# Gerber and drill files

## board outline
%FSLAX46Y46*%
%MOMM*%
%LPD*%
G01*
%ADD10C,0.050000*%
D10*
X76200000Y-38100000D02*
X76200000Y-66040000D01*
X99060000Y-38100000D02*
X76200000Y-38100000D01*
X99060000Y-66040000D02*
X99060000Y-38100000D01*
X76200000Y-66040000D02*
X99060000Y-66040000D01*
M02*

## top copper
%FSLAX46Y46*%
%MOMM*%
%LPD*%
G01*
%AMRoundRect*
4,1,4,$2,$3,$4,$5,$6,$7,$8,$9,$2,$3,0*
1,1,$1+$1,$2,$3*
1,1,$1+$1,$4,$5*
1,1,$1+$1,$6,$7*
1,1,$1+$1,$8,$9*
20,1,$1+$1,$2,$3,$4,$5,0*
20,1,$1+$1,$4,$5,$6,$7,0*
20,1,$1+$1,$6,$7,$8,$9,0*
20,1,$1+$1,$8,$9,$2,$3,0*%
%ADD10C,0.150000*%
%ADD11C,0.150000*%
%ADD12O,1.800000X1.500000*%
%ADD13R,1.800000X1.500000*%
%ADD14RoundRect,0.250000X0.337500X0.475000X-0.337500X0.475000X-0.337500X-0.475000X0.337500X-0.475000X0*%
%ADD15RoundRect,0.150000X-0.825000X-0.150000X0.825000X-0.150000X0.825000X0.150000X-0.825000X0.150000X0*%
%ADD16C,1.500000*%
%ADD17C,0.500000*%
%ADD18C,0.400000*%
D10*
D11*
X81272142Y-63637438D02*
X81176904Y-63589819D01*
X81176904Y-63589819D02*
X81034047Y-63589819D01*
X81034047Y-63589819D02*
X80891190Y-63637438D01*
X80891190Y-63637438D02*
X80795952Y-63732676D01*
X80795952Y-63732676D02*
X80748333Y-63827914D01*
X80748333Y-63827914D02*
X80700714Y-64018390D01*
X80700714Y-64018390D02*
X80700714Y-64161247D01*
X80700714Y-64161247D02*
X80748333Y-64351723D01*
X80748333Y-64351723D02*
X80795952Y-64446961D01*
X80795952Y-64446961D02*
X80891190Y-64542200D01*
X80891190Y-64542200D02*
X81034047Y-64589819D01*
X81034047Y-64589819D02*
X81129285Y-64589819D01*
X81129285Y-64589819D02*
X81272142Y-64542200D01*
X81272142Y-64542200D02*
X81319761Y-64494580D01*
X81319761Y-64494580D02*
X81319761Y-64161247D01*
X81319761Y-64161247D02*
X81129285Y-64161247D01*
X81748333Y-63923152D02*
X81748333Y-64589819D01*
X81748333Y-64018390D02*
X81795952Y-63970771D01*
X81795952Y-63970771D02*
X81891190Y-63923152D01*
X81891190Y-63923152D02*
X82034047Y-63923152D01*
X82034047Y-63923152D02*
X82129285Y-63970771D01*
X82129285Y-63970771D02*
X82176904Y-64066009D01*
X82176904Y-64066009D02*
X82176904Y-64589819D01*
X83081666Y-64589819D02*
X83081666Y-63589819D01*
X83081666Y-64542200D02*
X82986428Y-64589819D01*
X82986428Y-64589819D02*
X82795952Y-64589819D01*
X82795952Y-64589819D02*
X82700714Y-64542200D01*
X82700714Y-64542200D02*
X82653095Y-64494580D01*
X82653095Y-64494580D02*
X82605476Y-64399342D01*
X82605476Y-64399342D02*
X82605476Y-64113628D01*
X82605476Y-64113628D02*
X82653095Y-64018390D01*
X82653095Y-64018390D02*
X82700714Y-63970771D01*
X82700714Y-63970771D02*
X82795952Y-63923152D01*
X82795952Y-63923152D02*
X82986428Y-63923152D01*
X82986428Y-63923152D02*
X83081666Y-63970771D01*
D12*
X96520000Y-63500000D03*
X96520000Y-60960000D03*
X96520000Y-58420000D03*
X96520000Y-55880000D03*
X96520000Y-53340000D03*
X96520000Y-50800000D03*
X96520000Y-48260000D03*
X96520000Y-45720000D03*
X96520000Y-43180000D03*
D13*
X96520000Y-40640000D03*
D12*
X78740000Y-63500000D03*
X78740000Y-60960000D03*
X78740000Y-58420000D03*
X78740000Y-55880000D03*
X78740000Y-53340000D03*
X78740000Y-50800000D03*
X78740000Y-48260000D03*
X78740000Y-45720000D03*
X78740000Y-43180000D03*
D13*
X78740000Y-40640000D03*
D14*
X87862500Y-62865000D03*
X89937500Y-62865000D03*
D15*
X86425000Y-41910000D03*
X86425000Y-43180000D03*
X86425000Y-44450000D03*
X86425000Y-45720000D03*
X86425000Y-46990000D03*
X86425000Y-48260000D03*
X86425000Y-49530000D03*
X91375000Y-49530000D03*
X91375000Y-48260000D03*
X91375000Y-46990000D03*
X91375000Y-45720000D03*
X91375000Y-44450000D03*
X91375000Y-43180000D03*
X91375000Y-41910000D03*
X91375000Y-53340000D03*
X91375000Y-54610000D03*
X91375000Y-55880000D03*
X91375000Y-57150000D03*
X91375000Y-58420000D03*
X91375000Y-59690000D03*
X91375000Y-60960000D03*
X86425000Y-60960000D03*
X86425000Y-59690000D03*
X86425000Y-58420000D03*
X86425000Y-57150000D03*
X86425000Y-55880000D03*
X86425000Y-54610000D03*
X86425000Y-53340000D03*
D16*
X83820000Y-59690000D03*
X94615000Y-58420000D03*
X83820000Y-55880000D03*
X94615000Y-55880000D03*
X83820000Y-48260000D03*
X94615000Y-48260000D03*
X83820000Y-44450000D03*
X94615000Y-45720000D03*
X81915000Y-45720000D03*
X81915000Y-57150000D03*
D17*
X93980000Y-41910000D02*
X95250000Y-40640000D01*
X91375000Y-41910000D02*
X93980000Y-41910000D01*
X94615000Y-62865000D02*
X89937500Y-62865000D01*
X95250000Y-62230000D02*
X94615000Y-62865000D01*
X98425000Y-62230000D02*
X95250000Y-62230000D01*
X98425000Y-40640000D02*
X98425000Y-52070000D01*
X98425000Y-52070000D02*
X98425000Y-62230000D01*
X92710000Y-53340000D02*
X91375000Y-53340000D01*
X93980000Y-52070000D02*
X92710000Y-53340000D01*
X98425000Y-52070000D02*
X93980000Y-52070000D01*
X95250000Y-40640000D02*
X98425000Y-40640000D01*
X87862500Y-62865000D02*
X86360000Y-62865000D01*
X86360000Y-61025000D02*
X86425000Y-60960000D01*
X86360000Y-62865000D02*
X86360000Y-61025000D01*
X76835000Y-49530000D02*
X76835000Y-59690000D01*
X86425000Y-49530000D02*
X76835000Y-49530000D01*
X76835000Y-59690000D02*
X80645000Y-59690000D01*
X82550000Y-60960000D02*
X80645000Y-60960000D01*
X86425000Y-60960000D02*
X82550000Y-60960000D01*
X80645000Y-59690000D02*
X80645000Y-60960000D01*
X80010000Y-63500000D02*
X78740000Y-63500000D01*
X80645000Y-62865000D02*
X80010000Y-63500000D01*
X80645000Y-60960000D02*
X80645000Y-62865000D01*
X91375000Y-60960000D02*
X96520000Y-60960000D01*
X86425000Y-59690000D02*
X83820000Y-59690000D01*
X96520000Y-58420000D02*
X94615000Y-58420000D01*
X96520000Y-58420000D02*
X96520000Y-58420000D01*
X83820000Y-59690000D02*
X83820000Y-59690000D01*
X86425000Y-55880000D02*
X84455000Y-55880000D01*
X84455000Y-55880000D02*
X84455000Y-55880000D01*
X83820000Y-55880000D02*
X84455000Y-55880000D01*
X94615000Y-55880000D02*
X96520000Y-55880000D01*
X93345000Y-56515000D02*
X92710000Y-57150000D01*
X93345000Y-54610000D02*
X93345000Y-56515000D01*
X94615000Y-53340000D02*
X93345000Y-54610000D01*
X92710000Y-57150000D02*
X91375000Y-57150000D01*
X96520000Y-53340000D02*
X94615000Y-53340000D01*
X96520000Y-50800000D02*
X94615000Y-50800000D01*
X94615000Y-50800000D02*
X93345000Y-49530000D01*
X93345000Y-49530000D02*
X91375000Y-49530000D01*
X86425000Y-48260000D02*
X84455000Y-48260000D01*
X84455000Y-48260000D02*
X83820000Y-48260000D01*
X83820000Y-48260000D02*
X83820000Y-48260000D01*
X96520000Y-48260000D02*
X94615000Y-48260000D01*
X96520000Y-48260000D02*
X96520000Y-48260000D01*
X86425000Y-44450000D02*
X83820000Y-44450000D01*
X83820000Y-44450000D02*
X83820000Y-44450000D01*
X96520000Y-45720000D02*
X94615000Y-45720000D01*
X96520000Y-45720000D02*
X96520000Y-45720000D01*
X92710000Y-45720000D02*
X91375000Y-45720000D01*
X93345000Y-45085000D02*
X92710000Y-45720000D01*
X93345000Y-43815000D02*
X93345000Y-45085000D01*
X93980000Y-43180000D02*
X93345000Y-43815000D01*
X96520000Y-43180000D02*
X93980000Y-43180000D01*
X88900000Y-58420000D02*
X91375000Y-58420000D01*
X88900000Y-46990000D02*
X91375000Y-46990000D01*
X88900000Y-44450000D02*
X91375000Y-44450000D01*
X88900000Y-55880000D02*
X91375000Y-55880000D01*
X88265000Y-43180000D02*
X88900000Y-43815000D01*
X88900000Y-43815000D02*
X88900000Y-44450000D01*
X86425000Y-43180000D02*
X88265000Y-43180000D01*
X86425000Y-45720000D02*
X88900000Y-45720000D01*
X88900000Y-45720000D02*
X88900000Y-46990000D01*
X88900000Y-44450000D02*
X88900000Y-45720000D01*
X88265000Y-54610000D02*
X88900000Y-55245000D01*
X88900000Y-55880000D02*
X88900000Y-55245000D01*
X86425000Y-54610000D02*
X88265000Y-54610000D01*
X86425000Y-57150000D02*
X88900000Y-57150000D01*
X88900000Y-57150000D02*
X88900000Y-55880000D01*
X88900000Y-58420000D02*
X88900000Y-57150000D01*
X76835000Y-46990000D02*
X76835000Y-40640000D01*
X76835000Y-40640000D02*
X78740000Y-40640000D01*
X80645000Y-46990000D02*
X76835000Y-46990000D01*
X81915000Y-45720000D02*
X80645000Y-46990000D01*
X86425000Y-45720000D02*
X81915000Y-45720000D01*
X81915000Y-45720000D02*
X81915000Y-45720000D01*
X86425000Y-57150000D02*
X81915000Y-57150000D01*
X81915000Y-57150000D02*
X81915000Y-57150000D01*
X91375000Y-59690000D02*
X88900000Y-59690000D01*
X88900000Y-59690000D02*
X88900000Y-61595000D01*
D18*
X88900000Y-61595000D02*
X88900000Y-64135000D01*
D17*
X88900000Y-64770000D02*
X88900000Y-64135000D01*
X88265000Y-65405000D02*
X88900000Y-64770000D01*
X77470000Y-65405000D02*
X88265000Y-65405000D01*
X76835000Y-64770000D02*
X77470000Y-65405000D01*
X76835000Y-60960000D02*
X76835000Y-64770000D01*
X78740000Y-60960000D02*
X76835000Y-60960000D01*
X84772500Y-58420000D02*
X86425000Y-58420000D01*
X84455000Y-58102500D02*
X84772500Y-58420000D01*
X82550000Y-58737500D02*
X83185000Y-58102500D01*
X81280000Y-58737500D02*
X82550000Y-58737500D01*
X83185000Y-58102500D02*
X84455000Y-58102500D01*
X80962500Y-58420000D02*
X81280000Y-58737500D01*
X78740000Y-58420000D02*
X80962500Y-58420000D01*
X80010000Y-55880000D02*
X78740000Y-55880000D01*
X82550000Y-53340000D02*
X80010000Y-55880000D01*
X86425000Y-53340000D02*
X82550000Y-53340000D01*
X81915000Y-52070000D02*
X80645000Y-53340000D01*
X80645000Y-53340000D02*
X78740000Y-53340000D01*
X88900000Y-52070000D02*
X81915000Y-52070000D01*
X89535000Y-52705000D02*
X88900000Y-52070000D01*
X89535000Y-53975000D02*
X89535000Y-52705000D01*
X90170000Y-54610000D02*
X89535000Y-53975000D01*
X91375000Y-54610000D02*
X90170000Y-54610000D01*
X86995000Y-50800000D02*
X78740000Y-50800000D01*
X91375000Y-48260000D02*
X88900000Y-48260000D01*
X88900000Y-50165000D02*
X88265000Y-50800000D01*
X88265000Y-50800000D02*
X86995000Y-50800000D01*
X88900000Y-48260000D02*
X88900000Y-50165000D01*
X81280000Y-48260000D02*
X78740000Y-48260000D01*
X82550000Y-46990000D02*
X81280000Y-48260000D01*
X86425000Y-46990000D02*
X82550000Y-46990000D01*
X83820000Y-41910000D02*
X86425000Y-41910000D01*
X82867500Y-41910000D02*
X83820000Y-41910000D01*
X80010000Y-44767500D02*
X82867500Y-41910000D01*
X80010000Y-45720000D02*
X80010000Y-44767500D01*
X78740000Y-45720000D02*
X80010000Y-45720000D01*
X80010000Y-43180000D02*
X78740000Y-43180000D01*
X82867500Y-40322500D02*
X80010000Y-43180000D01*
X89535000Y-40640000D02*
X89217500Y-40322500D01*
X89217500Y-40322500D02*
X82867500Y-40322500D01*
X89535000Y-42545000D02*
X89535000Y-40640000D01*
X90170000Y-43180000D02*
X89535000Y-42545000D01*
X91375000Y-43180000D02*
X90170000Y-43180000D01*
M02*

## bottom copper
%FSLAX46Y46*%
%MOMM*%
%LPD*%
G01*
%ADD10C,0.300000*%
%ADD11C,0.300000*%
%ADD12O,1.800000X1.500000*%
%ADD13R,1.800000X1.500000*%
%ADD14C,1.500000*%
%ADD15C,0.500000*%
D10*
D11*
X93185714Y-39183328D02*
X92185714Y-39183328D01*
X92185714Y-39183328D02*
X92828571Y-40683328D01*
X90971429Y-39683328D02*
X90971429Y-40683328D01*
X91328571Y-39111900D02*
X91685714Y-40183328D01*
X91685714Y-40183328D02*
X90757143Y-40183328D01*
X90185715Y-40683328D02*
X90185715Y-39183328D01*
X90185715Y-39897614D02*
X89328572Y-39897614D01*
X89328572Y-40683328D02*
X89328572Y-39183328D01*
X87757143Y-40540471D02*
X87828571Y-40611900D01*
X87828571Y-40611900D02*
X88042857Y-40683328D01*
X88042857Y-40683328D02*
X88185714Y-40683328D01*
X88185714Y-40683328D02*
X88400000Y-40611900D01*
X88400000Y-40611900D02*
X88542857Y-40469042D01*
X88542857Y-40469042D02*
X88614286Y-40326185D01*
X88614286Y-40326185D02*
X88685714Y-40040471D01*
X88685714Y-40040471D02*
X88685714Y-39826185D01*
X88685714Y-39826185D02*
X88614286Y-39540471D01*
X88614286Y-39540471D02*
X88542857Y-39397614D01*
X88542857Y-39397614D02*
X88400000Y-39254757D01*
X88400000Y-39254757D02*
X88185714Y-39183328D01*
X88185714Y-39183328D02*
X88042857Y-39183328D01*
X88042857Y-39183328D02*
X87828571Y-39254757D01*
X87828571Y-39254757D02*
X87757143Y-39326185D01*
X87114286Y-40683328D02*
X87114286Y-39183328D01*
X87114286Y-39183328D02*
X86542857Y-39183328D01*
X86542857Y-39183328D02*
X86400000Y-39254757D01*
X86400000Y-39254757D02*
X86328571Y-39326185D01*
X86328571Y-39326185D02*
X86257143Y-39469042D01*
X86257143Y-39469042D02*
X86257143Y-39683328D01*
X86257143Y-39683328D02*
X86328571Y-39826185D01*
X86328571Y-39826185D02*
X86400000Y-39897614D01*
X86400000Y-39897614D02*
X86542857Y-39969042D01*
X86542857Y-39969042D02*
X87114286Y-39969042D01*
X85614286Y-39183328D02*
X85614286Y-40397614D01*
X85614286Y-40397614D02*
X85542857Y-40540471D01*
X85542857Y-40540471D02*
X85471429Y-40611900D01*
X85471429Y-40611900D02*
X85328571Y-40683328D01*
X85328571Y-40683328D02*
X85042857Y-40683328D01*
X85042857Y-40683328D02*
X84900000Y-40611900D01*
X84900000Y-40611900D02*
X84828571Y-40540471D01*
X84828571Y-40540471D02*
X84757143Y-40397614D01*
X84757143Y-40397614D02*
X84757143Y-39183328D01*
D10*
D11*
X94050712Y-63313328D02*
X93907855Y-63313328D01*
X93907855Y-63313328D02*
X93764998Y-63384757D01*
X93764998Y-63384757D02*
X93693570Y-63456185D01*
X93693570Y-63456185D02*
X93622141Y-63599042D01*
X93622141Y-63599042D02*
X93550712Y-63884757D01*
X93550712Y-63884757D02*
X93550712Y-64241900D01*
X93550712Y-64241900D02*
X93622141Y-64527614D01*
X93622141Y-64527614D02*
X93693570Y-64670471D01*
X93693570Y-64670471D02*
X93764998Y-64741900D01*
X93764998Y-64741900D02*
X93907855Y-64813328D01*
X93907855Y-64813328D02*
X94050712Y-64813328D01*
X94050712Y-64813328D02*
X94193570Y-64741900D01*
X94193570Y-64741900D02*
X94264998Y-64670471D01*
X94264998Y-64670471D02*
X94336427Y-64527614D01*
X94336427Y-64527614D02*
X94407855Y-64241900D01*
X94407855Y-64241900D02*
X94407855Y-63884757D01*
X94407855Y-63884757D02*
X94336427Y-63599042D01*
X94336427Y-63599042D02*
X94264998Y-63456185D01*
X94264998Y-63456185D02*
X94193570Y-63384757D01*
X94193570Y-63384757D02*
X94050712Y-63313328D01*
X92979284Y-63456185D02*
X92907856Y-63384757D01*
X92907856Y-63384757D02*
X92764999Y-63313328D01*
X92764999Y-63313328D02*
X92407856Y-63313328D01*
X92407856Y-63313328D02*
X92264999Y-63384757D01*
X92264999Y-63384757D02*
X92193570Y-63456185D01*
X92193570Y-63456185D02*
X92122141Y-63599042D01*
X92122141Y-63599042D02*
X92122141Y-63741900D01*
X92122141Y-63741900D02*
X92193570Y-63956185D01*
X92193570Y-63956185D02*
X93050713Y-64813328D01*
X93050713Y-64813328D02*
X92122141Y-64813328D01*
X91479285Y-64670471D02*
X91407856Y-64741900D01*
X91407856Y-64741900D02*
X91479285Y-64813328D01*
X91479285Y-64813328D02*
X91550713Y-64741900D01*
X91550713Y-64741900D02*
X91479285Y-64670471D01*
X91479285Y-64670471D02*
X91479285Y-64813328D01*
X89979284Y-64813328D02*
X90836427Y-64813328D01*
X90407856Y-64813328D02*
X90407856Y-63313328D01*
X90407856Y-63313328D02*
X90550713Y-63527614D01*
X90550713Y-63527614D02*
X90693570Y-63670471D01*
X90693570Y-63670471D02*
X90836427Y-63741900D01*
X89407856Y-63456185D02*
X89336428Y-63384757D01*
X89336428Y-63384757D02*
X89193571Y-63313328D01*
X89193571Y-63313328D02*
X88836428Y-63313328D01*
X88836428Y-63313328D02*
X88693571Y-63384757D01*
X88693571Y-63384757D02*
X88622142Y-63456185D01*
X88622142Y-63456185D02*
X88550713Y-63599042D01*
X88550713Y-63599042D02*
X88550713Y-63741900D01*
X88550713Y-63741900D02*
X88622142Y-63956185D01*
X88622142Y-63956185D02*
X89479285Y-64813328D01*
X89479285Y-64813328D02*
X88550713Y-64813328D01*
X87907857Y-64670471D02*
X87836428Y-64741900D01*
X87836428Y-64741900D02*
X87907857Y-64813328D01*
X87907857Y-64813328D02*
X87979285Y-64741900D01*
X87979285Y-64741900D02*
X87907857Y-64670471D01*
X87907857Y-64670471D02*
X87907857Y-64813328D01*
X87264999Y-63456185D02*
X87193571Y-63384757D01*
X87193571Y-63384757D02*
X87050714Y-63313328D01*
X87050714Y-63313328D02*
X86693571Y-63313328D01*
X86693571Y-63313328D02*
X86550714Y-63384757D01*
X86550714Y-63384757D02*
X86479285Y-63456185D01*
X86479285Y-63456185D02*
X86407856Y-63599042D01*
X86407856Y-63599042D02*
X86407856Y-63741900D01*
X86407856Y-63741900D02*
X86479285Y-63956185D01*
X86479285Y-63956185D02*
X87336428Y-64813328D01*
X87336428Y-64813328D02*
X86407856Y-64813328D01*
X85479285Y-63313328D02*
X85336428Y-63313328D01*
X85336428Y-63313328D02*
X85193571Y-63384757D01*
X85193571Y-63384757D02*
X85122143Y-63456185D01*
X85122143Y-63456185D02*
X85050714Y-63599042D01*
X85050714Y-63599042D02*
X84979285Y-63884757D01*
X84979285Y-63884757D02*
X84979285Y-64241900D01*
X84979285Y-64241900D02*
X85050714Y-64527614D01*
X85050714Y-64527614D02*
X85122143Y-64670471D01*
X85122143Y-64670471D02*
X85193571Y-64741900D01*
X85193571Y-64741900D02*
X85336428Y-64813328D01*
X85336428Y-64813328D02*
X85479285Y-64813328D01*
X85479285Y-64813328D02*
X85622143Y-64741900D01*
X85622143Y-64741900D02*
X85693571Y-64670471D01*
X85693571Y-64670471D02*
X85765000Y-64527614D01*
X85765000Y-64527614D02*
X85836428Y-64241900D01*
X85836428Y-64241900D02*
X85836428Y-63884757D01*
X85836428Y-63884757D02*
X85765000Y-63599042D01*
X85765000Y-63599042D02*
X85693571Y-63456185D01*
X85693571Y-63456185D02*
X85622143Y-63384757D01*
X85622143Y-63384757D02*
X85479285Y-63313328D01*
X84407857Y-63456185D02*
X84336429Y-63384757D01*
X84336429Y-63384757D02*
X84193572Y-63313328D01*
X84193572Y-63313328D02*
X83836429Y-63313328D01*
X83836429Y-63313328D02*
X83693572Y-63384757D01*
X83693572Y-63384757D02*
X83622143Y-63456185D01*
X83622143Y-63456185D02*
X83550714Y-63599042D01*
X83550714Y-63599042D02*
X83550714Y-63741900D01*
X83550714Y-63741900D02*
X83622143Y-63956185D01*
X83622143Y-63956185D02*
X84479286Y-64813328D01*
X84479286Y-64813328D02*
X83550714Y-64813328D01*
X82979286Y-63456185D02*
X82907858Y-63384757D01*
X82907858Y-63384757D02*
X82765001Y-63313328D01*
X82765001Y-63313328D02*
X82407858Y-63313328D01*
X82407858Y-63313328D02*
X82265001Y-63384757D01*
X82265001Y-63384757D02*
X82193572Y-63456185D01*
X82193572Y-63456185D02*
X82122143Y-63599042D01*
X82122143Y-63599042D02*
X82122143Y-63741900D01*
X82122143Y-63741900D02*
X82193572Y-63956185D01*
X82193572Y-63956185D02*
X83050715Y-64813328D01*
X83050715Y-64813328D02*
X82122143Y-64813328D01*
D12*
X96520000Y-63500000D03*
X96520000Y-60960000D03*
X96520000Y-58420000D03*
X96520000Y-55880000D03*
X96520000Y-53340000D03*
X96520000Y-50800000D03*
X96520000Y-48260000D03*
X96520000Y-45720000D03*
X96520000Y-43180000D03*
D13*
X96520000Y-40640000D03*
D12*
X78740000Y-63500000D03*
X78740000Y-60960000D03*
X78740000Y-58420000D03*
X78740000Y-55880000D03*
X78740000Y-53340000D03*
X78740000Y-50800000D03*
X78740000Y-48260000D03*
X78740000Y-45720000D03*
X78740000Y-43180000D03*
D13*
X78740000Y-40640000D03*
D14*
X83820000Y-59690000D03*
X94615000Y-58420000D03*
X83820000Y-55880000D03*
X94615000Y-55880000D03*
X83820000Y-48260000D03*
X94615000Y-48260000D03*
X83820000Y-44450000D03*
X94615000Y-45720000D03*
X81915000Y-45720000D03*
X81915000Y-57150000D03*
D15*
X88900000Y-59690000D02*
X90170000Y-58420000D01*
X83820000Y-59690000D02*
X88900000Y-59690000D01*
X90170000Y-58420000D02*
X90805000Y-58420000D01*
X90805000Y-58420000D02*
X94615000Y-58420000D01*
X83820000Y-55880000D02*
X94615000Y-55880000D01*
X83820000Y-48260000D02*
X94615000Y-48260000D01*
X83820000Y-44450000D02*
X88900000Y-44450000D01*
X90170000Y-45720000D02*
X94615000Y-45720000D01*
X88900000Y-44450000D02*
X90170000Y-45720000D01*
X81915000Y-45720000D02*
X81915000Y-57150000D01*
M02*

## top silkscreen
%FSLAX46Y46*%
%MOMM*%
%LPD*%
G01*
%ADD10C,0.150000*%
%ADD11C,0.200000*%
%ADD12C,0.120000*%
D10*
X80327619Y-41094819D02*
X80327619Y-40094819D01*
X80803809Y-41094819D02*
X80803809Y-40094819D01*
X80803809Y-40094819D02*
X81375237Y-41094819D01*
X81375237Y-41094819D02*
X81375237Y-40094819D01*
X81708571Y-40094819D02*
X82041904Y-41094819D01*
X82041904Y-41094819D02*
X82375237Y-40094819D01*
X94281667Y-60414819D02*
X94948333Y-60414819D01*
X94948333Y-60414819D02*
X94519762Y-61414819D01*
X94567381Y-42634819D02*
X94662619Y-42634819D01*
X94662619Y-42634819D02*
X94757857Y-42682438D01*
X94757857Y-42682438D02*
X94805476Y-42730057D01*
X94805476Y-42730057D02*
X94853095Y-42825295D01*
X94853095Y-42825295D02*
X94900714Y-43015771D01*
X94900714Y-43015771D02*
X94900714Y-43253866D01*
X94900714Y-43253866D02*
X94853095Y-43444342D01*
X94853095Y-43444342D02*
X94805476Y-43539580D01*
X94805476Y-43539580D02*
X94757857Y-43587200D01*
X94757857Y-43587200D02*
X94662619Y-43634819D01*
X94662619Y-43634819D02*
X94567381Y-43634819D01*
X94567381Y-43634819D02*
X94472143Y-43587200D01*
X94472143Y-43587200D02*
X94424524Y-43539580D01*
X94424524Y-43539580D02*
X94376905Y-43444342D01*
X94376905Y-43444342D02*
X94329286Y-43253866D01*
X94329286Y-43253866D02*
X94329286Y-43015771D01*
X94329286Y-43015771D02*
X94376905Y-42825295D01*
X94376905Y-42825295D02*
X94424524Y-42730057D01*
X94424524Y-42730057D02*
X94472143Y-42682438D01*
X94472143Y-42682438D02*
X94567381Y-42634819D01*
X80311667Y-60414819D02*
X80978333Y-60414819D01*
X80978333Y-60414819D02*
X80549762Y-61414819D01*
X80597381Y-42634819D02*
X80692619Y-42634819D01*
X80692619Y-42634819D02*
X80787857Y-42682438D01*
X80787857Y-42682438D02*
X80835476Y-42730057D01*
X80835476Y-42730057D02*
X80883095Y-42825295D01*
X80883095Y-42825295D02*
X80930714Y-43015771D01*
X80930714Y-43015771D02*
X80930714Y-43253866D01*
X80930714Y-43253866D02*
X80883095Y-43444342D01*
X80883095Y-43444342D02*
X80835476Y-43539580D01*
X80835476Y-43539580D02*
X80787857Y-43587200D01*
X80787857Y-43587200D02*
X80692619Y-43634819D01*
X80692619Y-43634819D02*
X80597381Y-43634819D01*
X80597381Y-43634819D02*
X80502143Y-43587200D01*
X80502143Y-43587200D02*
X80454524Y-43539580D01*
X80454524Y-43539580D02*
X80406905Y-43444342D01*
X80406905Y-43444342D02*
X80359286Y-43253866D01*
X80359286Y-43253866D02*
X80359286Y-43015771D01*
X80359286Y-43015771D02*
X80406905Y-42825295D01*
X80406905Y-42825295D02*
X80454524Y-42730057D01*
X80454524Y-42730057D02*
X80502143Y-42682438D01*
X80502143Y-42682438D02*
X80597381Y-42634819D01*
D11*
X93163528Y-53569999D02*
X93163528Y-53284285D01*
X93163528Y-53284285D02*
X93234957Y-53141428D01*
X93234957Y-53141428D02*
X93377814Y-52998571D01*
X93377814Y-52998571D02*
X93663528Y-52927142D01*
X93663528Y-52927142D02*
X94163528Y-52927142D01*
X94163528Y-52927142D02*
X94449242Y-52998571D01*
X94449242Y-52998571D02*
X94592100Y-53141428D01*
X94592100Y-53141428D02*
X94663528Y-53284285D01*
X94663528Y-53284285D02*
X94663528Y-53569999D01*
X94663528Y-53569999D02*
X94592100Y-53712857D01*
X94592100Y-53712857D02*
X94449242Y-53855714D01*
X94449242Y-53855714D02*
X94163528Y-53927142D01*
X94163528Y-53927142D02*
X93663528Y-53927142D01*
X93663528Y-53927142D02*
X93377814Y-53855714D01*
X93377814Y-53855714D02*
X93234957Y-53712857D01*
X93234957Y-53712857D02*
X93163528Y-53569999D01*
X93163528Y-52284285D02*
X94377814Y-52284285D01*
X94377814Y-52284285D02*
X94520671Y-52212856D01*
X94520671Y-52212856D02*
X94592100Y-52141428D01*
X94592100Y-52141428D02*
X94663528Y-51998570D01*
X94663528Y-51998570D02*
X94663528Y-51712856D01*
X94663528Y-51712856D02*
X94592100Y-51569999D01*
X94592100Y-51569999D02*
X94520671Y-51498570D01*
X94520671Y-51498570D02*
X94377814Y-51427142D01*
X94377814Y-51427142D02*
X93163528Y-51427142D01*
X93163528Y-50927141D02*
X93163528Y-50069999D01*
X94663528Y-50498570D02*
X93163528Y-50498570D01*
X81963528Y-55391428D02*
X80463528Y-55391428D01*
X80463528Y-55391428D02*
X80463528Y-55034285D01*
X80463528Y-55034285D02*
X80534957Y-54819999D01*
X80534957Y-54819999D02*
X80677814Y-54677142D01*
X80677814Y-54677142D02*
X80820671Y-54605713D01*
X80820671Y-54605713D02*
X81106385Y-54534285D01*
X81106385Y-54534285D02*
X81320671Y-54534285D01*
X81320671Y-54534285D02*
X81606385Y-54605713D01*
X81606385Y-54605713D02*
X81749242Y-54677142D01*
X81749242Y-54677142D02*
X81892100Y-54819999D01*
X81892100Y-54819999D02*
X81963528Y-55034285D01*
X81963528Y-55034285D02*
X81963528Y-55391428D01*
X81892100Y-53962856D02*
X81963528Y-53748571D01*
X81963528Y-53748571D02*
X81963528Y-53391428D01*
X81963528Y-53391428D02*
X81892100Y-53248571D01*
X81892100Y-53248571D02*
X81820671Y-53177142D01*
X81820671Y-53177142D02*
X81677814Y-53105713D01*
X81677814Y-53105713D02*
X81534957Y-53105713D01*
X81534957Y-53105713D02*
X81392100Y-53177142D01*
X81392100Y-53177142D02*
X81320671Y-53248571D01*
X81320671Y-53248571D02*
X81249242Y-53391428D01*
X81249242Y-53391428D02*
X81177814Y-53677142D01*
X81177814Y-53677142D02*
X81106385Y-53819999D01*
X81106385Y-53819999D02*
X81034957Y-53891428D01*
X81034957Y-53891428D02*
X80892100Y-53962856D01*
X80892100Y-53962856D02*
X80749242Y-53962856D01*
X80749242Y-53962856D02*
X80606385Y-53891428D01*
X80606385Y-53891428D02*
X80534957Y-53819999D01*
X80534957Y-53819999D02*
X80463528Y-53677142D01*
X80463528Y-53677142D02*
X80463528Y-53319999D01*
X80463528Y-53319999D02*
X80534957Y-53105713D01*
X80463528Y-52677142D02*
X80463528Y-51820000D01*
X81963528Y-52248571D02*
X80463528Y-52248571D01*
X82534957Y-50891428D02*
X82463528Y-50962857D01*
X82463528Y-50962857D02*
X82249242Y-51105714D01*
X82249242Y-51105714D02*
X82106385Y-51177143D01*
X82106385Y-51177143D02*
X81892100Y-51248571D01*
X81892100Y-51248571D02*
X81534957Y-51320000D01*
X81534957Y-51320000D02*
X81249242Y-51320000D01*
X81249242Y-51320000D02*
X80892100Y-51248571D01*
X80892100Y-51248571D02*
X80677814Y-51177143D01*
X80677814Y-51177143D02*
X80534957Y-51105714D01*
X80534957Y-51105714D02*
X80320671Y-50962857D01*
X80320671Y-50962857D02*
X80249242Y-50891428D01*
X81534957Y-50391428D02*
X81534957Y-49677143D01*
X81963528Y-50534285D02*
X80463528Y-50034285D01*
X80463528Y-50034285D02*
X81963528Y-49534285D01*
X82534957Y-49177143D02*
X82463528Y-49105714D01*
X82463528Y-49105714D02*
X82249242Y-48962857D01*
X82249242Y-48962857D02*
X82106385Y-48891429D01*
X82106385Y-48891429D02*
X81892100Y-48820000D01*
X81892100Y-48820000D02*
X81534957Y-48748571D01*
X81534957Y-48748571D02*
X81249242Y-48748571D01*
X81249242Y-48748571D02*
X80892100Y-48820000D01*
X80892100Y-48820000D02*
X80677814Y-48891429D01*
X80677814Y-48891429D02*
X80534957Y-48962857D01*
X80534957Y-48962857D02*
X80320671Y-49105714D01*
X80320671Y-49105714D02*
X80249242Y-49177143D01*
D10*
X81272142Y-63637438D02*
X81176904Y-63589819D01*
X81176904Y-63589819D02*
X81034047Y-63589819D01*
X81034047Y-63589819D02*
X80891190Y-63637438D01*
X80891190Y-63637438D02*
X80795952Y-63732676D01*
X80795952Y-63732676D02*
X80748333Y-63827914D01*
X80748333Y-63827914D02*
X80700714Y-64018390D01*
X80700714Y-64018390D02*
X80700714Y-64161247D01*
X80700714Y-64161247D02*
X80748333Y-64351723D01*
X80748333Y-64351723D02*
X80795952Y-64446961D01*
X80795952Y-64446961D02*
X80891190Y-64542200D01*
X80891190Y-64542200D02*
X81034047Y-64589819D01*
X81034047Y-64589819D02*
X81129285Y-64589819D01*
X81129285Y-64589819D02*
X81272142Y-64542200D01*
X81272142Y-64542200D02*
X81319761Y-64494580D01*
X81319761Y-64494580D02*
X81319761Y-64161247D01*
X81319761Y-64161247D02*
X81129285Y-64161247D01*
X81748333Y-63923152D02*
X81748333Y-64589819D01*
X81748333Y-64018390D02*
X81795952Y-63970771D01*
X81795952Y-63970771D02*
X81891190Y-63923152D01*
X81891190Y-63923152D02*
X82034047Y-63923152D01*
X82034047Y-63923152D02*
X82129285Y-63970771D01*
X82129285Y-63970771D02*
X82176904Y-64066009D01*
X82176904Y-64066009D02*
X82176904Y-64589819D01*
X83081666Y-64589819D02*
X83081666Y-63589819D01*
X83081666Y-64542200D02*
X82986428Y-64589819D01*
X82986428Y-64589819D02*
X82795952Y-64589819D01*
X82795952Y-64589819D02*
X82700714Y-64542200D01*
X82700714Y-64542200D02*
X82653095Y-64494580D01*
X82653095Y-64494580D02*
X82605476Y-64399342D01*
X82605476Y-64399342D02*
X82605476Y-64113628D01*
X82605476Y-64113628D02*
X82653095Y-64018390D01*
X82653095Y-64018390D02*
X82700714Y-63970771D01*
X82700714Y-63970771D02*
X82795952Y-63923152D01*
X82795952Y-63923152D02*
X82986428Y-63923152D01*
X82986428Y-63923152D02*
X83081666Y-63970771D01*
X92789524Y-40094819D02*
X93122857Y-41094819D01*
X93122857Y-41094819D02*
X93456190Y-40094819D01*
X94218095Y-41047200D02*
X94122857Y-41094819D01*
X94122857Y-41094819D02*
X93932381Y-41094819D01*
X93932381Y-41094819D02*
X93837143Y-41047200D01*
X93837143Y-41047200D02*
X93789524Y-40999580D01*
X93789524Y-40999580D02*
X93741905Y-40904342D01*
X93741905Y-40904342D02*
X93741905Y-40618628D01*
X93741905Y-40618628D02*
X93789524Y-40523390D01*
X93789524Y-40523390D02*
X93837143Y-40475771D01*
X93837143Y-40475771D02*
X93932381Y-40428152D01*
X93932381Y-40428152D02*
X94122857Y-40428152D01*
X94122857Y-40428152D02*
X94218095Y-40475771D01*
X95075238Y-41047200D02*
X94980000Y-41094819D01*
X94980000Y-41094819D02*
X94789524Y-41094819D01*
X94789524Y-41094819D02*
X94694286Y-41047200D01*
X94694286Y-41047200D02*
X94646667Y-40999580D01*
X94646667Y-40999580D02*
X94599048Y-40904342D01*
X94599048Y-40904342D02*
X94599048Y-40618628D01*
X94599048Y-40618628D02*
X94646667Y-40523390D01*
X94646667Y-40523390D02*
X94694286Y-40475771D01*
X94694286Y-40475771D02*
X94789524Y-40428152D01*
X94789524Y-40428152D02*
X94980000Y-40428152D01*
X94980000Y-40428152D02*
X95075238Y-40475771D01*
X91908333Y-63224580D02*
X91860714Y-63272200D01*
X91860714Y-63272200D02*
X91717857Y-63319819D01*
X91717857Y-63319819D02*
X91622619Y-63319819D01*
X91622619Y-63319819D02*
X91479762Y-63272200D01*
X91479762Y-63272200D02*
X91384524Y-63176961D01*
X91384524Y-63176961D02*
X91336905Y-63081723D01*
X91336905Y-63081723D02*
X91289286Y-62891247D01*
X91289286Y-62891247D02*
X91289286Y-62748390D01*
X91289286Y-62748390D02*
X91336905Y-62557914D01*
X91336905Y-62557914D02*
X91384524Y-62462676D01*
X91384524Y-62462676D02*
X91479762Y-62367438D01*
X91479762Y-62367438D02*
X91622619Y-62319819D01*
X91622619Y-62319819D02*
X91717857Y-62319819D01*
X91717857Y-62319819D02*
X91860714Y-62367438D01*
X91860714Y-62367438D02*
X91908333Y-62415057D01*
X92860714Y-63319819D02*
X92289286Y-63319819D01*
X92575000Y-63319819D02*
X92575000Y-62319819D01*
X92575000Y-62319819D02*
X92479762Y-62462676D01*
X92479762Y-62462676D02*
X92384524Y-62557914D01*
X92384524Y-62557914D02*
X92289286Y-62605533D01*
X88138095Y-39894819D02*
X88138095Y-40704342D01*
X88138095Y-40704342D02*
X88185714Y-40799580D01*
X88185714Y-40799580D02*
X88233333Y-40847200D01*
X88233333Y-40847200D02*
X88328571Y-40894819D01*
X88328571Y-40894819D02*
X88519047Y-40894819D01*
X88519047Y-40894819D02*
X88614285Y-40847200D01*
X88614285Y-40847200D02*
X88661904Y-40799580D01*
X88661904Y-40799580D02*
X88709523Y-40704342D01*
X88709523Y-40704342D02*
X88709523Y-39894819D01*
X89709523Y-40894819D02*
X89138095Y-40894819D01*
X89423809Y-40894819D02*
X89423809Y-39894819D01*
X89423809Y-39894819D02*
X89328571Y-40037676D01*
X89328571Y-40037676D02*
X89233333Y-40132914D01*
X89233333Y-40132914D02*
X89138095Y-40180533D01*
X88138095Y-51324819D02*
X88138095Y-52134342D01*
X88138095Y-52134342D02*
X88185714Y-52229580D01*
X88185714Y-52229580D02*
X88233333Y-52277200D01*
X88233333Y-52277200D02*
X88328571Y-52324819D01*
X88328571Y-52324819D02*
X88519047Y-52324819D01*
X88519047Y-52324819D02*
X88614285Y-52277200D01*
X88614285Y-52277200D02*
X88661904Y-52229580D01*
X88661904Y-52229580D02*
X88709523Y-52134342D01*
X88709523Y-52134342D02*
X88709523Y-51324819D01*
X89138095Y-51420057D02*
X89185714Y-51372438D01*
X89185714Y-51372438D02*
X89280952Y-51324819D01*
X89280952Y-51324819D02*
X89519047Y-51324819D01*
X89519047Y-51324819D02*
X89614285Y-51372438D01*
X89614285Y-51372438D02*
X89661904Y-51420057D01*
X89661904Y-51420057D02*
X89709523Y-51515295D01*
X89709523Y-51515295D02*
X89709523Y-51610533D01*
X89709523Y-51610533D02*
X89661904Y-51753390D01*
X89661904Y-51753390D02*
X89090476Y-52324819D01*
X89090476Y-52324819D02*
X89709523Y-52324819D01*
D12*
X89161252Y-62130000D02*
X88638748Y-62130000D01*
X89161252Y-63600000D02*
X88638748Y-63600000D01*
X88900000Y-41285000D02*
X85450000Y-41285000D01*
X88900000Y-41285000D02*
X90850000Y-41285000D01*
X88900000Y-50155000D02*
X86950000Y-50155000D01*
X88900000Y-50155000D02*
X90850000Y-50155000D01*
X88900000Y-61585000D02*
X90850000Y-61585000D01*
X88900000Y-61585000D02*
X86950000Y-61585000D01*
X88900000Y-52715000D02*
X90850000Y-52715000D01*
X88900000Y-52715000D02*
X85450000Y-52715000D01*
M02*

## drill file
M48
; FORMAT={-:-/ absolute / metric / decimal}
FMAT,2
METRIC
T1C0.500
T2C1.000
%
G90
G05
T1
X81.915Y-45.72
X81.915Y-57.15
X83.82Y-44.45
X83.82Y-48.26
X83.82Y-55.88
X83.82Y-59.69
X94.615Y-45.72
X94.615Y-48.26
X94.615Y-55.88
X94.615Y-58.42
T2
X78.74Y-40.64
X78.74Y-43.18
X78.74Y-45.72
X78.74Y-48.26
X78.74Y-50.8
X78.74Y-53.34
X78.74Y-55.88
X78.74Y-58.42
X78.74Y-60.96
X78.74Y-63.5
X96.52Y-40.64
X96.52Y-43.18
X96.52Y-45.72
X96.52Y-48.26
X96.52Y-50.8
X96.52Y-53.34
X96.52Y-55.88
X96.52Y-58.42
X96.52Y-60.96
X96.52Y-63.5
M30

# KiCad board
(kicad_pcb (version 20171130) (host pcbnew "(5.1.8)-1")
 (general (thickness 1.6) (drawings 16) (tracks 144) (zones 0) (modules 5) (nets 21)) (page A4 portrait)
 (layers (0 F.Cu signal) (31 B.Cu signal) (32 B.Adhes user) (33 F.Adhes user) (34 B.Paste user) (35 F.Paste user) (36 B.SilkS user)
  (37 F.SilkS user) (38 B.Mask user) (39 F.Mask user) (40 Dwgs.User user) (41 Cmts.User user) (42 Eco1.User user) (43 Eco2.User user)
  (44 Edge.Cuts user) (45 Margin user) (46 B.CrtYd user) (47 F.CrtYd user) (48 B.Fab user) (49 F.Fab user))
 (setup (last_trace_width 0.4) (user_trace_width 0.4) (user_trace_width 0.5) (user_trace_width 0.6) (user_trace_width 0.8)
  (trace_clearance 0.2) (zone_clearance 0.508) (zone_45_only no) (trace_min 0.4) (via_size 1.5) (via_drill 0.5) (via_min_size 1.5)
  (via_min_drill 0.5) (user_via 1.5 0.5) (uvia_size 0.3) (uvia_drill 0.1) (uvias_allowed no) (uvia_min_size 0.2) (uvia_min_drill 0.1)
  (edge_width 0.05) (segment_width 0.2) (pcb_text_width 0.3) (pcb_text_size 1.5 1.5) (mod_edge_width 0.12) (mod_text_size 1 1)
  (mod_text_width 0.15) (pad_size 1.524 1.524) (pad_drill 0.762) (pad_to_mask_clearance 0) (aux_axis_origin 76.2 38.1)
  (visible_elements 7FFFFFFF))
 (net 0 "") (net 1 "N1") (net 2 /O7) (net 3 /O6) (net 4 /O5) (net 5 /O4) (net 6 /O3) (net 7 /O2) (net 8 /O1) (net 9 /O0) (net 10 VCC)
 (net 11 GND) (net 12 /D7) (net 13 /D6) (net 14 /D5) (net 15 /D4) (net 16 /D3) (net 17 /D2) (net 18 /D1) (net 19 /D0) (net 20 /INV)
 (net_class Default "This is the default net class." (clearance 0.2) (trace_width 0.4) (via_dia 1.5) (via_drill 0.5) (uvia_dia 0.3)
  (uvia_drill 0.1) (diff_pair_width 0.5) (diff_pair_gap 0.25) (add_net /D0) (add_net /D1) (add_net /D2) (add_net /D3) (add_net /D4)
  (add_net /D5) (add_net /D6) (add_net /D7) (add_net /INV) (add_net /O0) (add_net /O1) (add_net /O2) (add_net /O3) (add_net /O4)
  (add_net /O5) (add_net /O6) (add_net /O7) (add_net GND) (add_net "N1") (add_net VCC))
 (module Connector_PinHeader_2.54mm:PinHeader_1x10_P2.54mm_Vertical (layer B.Cu) (at 96.52 40.64 180)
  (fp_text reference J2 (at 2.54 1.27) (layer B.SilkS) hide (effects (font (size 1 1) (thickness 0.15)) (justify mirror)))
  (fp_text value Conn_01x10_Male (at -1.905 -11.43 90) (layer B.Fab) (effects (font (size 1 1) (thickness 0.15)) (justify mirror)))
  (pad 10 thru_hole oval (at 0 -22.86 180) (size 1.8 1.5) (drill 1) (layers *.Cu *.Mask) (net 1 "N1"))
  (pad 9 thru_hole oval (at 0 -20.32 180) (size 1.8 1.5) (drill 1) (layers *.Cu *.Mask) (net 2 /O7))
  (pad 8 thru_hole oval (at 0 -17.78 180) (size 1.8 1.5) (drill 1) (layers *.Cu *.Mask) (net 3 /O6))
  (pad 7 thru_hole oval (at 0 -15.24 180) (size 1.8 1.5) (drill 1) (layers *.Cu *.Mask) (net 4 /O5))
  (pad 6 thru_hole oval (at 0 -12.7 180) (size 1.8 1.5) (drill 1) (layers *.Cu *.Mask) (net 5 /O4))
  (pad 5 thru_hole oval (at 0 -10.16 180) (size 1.8 1.5) (drill 1) (layers *.Cu *.Mask) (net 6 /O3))
  (pad 4 thru_hole oval (at 0 -7.62 180) (size 1.8 1.5) (drill 1) (layers *.Cu *.Mask) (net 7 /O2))
  (pad 3 thru_hole oval (at 0 -5.08 180) (size 1.8 1.5) (drill 1) (layers *.Cu *.Mask) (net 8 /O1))
  (pad 2 thru_hole oval (at 0 -2.54 180) (size 1.8 1.5) (drill 1) (layers *.Cu *.Mask) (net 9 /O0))
  (pad 1 thru_hole rect (at 0 0 180) (size 1.8 1.5) (drill 1) (layers *.Cu *.Mask) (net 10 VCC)))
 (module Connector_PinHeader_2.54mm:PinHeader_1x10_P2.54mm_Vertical (layer B.Cu) (at 78.74 40.64 180)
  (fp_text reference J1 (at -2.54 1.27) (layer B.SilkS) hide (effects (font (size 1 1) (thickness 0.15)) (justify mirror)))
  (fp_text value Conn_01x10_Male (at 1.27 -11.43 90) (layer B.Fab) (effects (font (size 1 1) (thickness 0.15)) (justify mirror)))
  (pad 10 thru_hole oval (at 0 -22.86 180) (size 1.8 1.5) (drill 1) (layers *.Cu *.Mask) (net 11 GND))
  (pad 9 thru_hole oval (at 0 -20.32 180) (size 1.8 1.5) (drill 1) (layers *.Cu *.Mask) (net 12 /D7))
  (pad 8 thru_hole oval (at 0 -17.78 180) (size 1.8 1.5) (drill 1) (layers *.Cu *.Mask) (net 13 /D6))
  (pad 7 thru_hole oval (at 0 -15.24 180) (size 1.8 1.5) (drill 1) (layers *.Cu *.Mask) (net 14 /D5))
  (pad 6 thru_hole oval (at 0 -12.7 180) (size 1.8 1.5) (drill 1) (layers *.Cu *.Mask) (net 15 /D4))
  (pad 5 thru_hole oval (at 0 -10.16 180) (size 1.8 1.5) (drill 1) (layers *.Cu *.Mask) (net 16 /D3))
  (pad 4 thru_hole oval (at 0 -7.62 180) (size 1.8 1.5) (drill 1) (layers *.Cu *.Mask) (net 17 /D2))
  (pad 3 thru_hole oval (at 0 -5.08 180) (size 1.8 1.5) (drill 1) (layers *.Cu *.Mask) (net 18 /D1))
  (pad 2 thru_hole oval (at 0 -2.54 180) (size 1.8 1.5) (drill 1) (layers *.Cu *.Mask) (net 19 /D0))
  (pad 1 thru_hole rect (at 0 0 180) (size 1.8 1.5) (drill 1) (layers *.Cu *.Mask) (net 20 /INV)))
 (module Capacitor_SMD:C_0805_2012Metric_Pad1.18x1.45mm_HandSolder (layer F.Cu) (at 88.9 62.865 180)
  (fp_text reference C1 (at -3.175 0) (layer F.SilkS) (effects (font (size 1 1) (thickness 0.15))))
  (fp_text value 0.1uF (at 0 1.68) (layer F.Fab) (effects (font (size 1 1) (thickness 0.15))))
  (fp_line (start -0.261252 0.735) (end 0.261252 0.735) (layer F.SilkS) (width 0.12))
  (fp_line (start -0.261252 -0.735) (end 0.261252 -0.735) (layer F.SilkS) (width 0.12))
  (pad 2 smd roundrect (at 1.0375 0 180) (size 1.175 1.45) (layers F.Cu F.Paste F.Mask) (roundrect_rratio 0.2127659574468085) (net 11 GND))
  (pad 1 smd roundrect (at -1.0375 0 180) (size 1.175 1.45) (layers F.Cu F.Paste F.Mask) (roundrect_rratio 0.2127659574468085) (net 10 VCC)))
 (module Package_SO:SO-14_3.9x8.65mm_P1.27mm (layer F.Cu) (at 88.9 45.72)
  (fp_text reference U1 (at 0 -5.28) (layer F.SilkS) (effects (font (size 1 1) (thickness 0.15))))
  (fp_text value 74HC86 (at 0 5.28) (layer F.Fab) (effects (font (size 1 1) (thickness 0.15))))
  (fp_line (start 0 -4.435) (end -3.45 -4.435) (layer F.SilkS) (width 0.12))
  (fp_line (start 0 -4.435) (end 1.95 -4.435) (layer F.SilkS) (width 0.12))
  (fp_line (start 0 4.435) (end -1.95 4.435) (layer F.SilkS) (width 0.12))
  (fp_line (start 0 4.435) (end 1.95 4.435) (layer F.SilkS) (width 0.12))
  (pad 1 smd roundrect (at -2.475 -3.81) (size 1.95 0.6) (layers F.Cu F.Paste F.Mask) (roundrect_rratio 0.25) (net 18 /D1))
  (pad 2 smd roundrect (at -2.475 -2.54) (size 1.95 0.6) (layers F.Cu F.Paste F.Mask) (roundrect_rratio 0.25) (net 20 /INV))
  (pad 3 smd roundrect (at -2.475 -1.27) (size 1.95 0.6) (layers F.Cu F.Paste F.Mask) (roundrect_rratio 0.25) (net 8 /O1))
  (pad 4 smd roundrect (at -2.475 0) (size 1.95 0.6) (layers F.Cu F.Paste F.Mask) (roundrect_rratio 0.25) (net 20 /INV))
  (pad 5 smd roundrect (at -2.475 1.27) (size 1.95 0.6) (layers F.Cu F.Paste F.Mask) (roundrect_rratio 0.25) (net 17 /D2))
  (pad 6 smd roundrect (at -2.475 2.54) (size 1.95 0.6) (layers F.Cu F.Paste F.Mask) (roundrect_rratio 0.25) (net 7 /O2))
  (pad 7 smd roundrect (at -2.475 3.81) (size 1.95 0.6) (layers F.Cu F.Paste F.Mask) (roundrect_rratio 0.25) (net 11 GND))
  (pad 8 smd roundrect (at 2.475 3.81) (size 1.95 0.6) (layers F.Cu F.Paste F.Mask) (roundrect_rratio 0.25) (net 6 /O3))
  (pad 9 smd roundrect (at 2.475 2.54) (size 1.95 0.6) (layers F.Cu F.Paste F.Mask) (roundrect_rratio 0.25) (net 16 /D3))
  (pad 10 smd roundrect (at 2.475 1.27) (size 1.95 0.6) (layers F.Cu F.Paste F.Mask) (roundrect_rratio 0.25) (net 20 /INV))
  (pad 11 smd roundrect (at 2.475 0) (size 1.95 0.6) (layers F.Cu F.Paste F.Mask) (roundrect_rratio 0.25) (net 9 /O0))
  (pad 12 smd roundrect (at 2.475 -1.27) (size 1.95 0.6) (layers F.Cu F.Paste F.Mask) (roundrect_rratio 0.25) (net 20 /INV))
  (pad 13 smd roundrect (at 2.475 -2.54) (size 1.95 0.6) (layers F.Cu F.Paste F.Mask) (roundrect_rratio 0.25) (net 19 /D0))
  (pad 14 smd roundrect (at 2.475 -3.81) (size 1.95 0.6) (layers F.Cu F.Paste F.Mask) (roundrect_rratio 0.25) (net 10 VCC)))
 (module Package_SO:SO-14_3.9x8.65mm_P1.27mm (layer F.Cu) (at 88.9 57.15)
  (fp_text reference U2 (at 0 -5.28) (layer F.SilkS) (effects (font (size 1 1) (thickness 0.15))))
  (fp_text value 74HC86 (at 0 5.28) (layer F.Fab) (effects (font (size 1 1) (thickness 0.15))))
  (fp_line (start 0 4.435) (end 1.95 4.435) (layer F.SilkS) (width 0.12))
  (fp_line (start 0 4.435) (end -1.95 4.435) (layer F.SilkS) (width 0.12))
  (fp_line (start 0 -4.435) (end 1.95 -4.435) (layer F.SilkS) (width 0.12))
  (fp_line (start 0 -4.435) (end -3.45 -4.435) (layer F.SilkS) (width 0.12))
  (pad 14 smd roundrect (at 2.475 -3.81) (size 1.95 0.6) (layers F.Cu F.Paste F.Mask) (roundrect_rratio 0.25) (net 10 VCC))
  (pad 13 smd roundrect (at 2.475 -2.54) (size 1.95 0.6) (layers F.Cu F.Paste F.Mask) (roundrect_rratio 0.25) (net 15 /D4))
  (pad 12 smd roundrect (at 2.475 -1.27) (size 1.95 0.6) (layers F.Cu F.Paste F.Mask) (roundrect_rratio 0.25) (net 20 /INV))
  (pad 11 smd roundrect (at 2.475 0) (size 1.95 0.6) (layers F.Cu F.Paste F.Mask) (roundrect_rratio 0.25) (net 5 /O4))
  (pad 10 smd roundrect (at 2.475 1.27) (size 1.95 0.6) (layers F.Cu F.Paste F.Mask) (roundrect_rratio 0.25) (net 20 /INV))
  (pad 9 smd roundrect (at 2.475 2.54) (size 1.95 0.6) (layers F.Cu F.Paste F.Mask) (roundrect_rratio 0.25) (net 12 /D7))
  (pad 8 smd roundrect (at 2.475 3.81) (size 1.95 0.6) (layers F.Cu F.Paste F.Mask) (roundrect_rratio 0.25) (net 2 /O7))
  (pad 7 smd roundrect (at -2.475 3.81) (size 1.95 0.6) (layers F.Cu F.Paste F.Mask) (roundrect_rratio 0.25) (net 11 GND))
  (pad 6 smd roundrect (at -2.475 2.54) (size 1.95 0.6) (layers F.Cu F.Paste F.Mask) (roundrect_rratio 0.25) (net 3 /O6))
  (pad 5 smd roundrect (at -2.475 1.27) (size 1.95 0.6) (layers F.Cu F.Paste F.Mask) (roundrect_rratio 0.25) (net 13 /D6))
  (pad 4 smd roundrect (at -2.475 0) (size 1.95 0.6) (layers F.Cu F.Paste F.Mask) (roundrect_rratio 0.25) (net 20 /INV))
  (pad 3 smd roundrect (at -2.475 -1.27) (size 1.95 0.6) (layers F.Cu F.Paste F.Mask) (roundrect_rratio 0.25) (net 4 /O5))
  (pad 2 smd roundrect (at -2.475 -2.54) (size 1.95 0.6) (layers F.Cu F.Paste F.Mask) (roundrect_rratio 0.25) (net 20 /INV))
  (pad 1 smd roundrect (at -2.475 -3.81) (size 1.95 0.6) (layers F.Cu F.Paste F.Mask) (roundrect_rratio 0.25) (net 14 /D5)))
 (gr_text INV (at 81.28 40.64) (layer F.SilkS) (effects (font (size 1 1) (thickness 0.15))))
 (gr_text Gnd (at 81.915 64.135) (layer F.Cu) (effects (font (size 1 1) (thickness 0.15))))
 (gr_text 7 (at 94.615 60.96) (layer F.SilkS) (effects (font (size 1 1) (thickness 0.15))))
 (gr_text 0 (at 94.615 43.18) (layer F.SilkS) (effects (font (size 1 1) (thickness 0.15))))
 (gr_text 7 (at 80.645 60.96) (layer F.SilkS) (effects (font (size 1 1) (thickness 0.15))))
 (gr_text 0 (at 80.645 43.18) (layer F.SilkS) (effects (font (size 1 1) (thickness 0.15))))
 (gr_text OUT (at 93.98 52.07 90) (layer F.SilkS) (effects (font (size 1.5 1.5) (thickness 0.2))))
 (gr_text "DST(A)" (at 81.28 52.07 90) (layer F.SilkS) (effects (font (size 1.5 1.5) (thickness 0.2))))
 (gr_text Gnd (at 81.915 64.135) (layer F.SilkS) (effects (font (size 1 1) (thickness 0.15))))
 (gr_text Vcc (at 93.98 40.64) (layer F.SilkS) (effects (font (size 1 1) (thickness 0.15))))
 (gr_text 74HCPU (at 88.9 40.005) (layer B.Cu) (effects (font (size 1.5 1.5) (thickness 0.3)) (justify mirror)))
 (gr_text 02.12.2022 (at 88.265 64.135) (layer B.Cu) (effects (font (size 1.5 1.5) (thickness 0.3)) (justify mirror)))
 (gr_line (start 76.2 38.1) (end 76.2 66.04) (layer Edge.Cuts) (width 0.05))
 (gr_line (start 99.06 38.1) (end 76.2 38.1) (layer Edge.Cuts) (width 0.05))
 (gr_line (start 99.06 66.04) (end 99.06 38.1) (layer Edge.Cuts) (width 0.05))
 (gr_line (start 76.2 66.04) (end 99.06 66.04) (layer Edge.Cuts) (width 0.05))
 (segment (start 93.98 41.91) (end 95.25 40.64) (width 0.5) (layer F.Cu) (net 10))
 (segment (start 91.375 41.91) (end 93.98 41.91) (width 0.5) (layer F.Cu) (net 10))
 (segment (start 94.615 62.865) (end 89.9375 62.865) (width 0.5) (layer F.Cu) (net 10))
 (segment (start 95.25 62.23) (end 94.615 62.865) (width 0.5) (layer F.Cu) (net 10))
 (segment (start 98.425 62.23) (end 95.25 62.23) (width 0.5) (layer F.Cu) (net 10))
 (segment (start 98.425 40.64) (end 98.425 52.07) (width 0.5) (layer F.Cu) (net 10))
 (segment (start 98.425 52.07) (end 98.425 62.23) (width 0.5) (layer F.Cu) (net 10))
 (segment (start 92.71 53.34) (end 91.375 53.34) (width 0.5) (layer F.Cu) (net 10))
 (segment (start 93.98 52.07) (end 92.71 53.34) (width 0.5) (layer F.Cu) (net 10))
 (segment (start 98.425 52.07) (end 93.98 52.07) (width 0.5) (layer F.Cu) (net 10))
 (segment (start 95.25 40.64) (end 98.425 40.64) (width 0.5) (layer F.Cu) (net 10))
 (segment (start 87.8625 62.865) (end 86.36 62.865) (width 0.5) (layer F.Cu) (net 11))
 (segment (start 86.36 61.025) (end 86.425 60.96) (width 0.5) (layer F.Cu) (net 11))
 (segment (start 86.36 62.865) (end 86.36 61.025) (width 0.5) (layer F.Cu) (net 11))
 (segment (start 76.835 49.53) (end 76.835 59.69) (width 0.5) (layer F.Cu) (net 11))
 (segment (start 86.425 49.53) (end 76.835 49.53) (width 0.5) (layer F.Cu) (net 11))
 (segment (start 76.835 59.69) (end 80.645 59.69) (width 0.5) (layer F.Cu) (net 11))
 (segment (start 82.55 60.96) (end 80.645 60.96) (width 0.5) (layer F.Cu) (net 11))
 (segment (start 86.425 60.96) (end 82.55 60.96) (width 0.5) (layer F.Cu) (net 11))
 (segment (start 80.645 59.69) (end 80.645 60.96) (width 0.5) (layer F.Cu) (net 11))
 (segment (start 80.01 63.5) (end 78.74 63.5) (width 0.5) (layer F.Cu) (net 11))
 (segment (start 80.645 62.865) (end 80.01 63.5) (width 0.5) (layer F.Cu) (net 11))
 (segment (start 80.645 60.96) (end 80.645 62.865) (width 0.5) (layer F.Cu) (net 11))
 (segment (start 91.375 60.96) (end 96.52 60.96) (width 0.5) (layer F.Cu) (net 2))
 (segment (start 86.425 59.69) (end 83.82 59.69) (width 0.5) (layer F.Cu) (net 3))
 (segment (start 96.52 58.42) (end 94.615 58.42) (width 0.5) (layer F.Cu) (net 3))
 (segment (start 96.52 58.42) (end 96.52 58.42) (width 0.5) (layer F.Cu) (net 3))
 (segment (start 83.82 59.69) (end 83.82 59.69) (width 0.5) (layer F.Cu) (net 3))
 (via (at 83.82 59.69) (size 1.5) (drill 0.5) (layers F.Cu B.Cu) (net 3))
 (segment (start 88.9 59.69) (end 90.17 58.42) (width 0.5) (layer B.Cu) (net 3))
 (segment (start 83.82 59.69) (end 88.9 59.69) (width 0.5) (layer B.Cu) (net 3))
 (segment (start 90.17 58.42) (end 90.805 58.42) (width 0.5) (layer B.Cu) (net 3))
 (segment (start 90.805 58.42) (end 94.615 58.42) (width 0.5) (layer B.Cu) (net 3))
 (via (at 94.615 58.42) (size 1.5) (drill 0.5) (layers F.Cu B.Cu) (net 3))
 (segment (start 86.425 55.88) (end 84.455 55.88) (width 0.5) (layer F.Cu) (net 4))
 (segment (start 84.455 55.88) (end 84.455 55.88) (width 0.5) (layer F.Cu) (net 4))
 (via (at 83.82 55.88) (size 1.5) (drill 0.5) (layers F.Cu B.Cu) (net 4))
 (segment (start 83.82 55.88) (end 84.455 55.88) (width 0.5) (layer F.Cu) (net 4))
 (segment (start 94.615 55.88) (end 96.52 55.88) (width 0.5) (layer F.Cu) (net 4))
 (segment (start 83.82 55.88) (end 94.615 55.88) (width 0.5) (layer B.Cu) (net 4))
 (via (at 94.615 55.88) (size 1.5) (drill 0.5) (layers F.Cu B.Cu) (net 4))
 (segment (start 93.345 56.515) (end 92.71 57.15) (width 0.5) (layer F.Cu) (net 5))
 (segment (start 93.345 54.61) (end 93.345 56.515) (width 0.5) (layer F.Cu) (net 5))
 (segment (start 94.615 53.34) (end 93.345 54.61) (width 0.5) (layer F.Cu) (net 5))
 (segment (start 92.71 57.15) (end 91.375 57.15) (width 0.5) (layer F.Cu) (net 5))
 (segment (start 96.52 53.34) (end 94.615 53.34) (width 0.5) (layer F.Cu) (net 5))
 (segment (start 96.52 50.8) (end 94.615 50.8) (width 0.5) (layer F.Cu) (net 6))
 (segment (start 94.615 50.8) (end 93.345 49.53) (width 0.5) (layer F.Cu) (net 6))
 (segment (start 93.345 49.53) (end 91.375 49.53) (width 0.5) (layer F.Cu) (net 6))
 (segment (start 86.425 48.26) (end 84.455 48.26) (width 0.5) (layer F.Cu) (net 7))
 (segment (start 84.455 48.26) (end 83.82 48.26) (width 0.5) (layer F.Cu) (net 7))
 (segment (start 83.82 48.26) (end 83.82 48.26) (width 0.5) (layer F.Cu) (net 7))
 (via (at 83.82 48.26) (size 1.5) (drill 0.5) (layers F.Cu B.Cu) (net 7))
 (segment (start 96.52 48.26) (end 94.615 48.26) (width 0.5) (layer F.Cu) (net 7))
 (segment (start 96.52 48.26) (end 96.52 48.26) (width 0.5) (layer F.Cu) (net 7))
 (segment (start 83.82 48.26) (end 94.615 48.26) (width 0.5) (layer B.Cu) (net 7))
 (via (at 94.615 48.26) (size 1.5) (drill 0.5) (layers F.Cu B.Cu) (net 7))
 (segment (start 86.425 44.45) (end 83.82 44.45) (width 0.5) (layer F.Cu) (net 8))
 (segment (start 83.82 44.45) (end 83.82 44.45) (width 0.5) (layer F.Cu) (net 8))
 (via (at 83.82 44.45) (size 1.5) (drill 0.5) (layers F.Cu B.Cu) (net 8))
 (segment (start 96.52 45.72) (end 94.615 45.72) (width 0.5) (layer F.Cu) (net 8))
 (segment (start 96.52 45.72) (end 96.52 45.72) (width 0.5) (layer F.Cu) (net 8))
 (segment (start 83.82 44.45) (end 88.9 44.45) (width 0.5) (layer B.Cu) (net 8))
 (segment (start 90.17 45.72) (end 94.615 45.72) (width 0.5) (layer B.Cu) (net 8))
 (segment (start 88.9 44.45) (end 90.17 45.72) (width 0.5) (layer B.Cu) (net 8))
 (via (at 94.615 45.72) (size 1.5) (drill 0.5) (layers F.Cu B.Cu) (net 8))
 (segment (start 92.71 45.72) (end 91.375 45.72) (width 0.5) (layer F.Cu) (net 9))
 (segment (start 93.345 45.085) (end 92.71 45.72) (width 0.5) (layer F.Cu) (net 9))
 (segment (start 93.345 43.815) (end 93.345 45.085) (width 0.5) (layer F.Cu) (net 9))
 (segment (start 93.98 43.18) (end 93.345 43.815) (width 0.5) (layer F.Cu) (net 9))
 (segment (start 96.52 43.18) (end 93.98 43.18) (width 0.5) (layer F.Cu) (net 9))
 (segment (start 88.9 58.42) (end 91.375 58.42) (width 0.5) (layer F.Cu) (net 20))
 (segment (start 88.9 46.99) (end 91.375 46.99) (width 0.5) (layer F.Cu) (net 20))
 (segment (start 88.9 44.45) (end 91.375 44.45) (width 0.5) (layer F.Cu) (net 20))
 (segment (start 88.9 55.88) (end 91.375 55.88) (width 0.5) (layer F.Cu) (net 20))
 (segment (start 88.265 43.18) (end 88.9 43.815) (width 0.5) (layer F.Cu) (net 20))
 (segment (start 88.9 43.815) (end 88.9 44.45) (width 0.5) (layer F.Cu) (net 20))
 (segment (start 86.425 43.18) (end 88.265 43.18) (width 0.5) (layer F.Cu) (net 20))
 (segment (start 86.425 45.72) (end 88.9 45.72) (width 0.5) (layer F.Cu) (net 20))
 (segment (start 88.9 45.72) (end 88.9 46.99) (width 0.5) (layer F.Cu) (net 20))
 (segment (start 88.9 44.45) (end 88.9 45.72) (width 0.5) (layer F.Cu) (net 20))
 (segment (start 88.265 54.61) (end 88.9 55.245) (width 0.5) (layer F.Cu) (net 20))
 (segment (start 88.9 55.88) (end 88.9 55.245) (width 0.5) (layer F.Cu) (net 20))
 (segment (start 86.425 54.61) (end 88.265 54.61) (width 0.5) (layer F.Cu) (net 20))
 (segment (start 86.425 57.15) (end 88.9 57.15) (width 0.5) (layer F.Cu) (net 20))
 (segment (start 88.9 57.15) (end 88.9 55.88) (width 0.5) (layer F.Cu) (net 20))
 (segment (start 88.9 58.42) (end 88.9 57.15) (width 0.5) (layer F.Cu) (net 20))
 (segment (start 76.835 46.99) (end 76.835 40.64) (width 0.5) (layer F.Cu) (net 20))
 (segment (start 76.835 40.64) (end 78.74 40.64) (width 0.5) (layer F.Cu) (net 20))
 (segment (start 80.645 46.99) (end 76.835 46.99) (width 0.5) (layer F.Cu) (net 20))
 (segment (start 81.915 45.72) (end 80.645 46.99) (width 0.5) (layer F.Cu) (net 20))
 (segment (start 86.425 45.72) (end 81.915 45.72) (width 0.5) (layer F.Cu) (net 20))
 (segment (start 81.915 45.72) (end 81.915 45.72) (width 0.5) (layer F.Cu) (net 20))
 (via (at 81.915 45.72) (size 1.5) (drill 0.5) (layers F.Cu B.Cu) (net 20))
 (segment (start 86.425 57.15) (end 81.915 57.15) (width 0.5) (layer F.Cu) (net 20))
 (segment (start 81.915 57.15) (end 81.915 57.15) (width 0.5) (layer F.Cu) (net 20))
 (via (at 81.915 57.15) (size 1.5) (drill 0.5) (layers F.Cu B.Cu) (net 20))
 (segment (start 81.915 45.72) (end 81.915 57.15) (width 0.5) (layer B.Cu) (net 20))
 (segment (start 91.375 59.69) (end 88.9 59.69) (width 0.5) (layer F.Cu) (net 12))
 (segment (start 88.9 59.69) (end 88.9 61.595) (width 0.5) (layer F.Cu) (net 12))
 (segment (start 88.9 61.595) (end 88.9 64.135) (width 0.4) (layer F.Cu) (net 12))
 (segment (start 88.9 64.77) (end 88.9 64.135) (width 0.5) (layer F.Cu) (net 12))
 (segment (start 88.265 65.405) (end 88.9 64.77) (width 0.5) (layer F.Cu) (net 12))
 (segment (start 77.47 65.405) (end 88.265 65.405) (width 0.5) (layer F.Cu) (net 12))
 (segment (start 76.835 64.77) (end 77.47 65.405) (width 0.5) (layer F.Cu) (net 12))
 (segment (start 76.835 60.96) (end 76.835 64.77) (width 0.5) (layer F.Cu) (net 12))
 (segment (start 78.74 60.96) (end 76.835 60.96) (width 0.5) (layer F.Cu) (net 12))
 (segment (start 84.7725 58.42) (end 86.425 58.42) (width 0.5) (layer F.Cu) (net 13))
 (segment (start 84.455 58.1025) (end 84.7725 58.42) (width 0.5) (layer F.Cu) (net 13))
 (segment (start 82.55 58.7375) (end 83.185 58.1025) (width 0.5) (layer F.Cu) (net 13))
 (segment (start 81.28 58.7375) (end 82.55 58.7375) (width 0.5) (layer F.Cu) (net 13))
 (segment (start 83.185 58.1025) (end 84.455 58.1025) (width 0.5) (layer F.Cu) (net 13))
 (segment (start 80.9625 58.42) (end 81.28 58.7375) (width 0.5) (layer F.Cu) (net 13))
 (segment (start 78.74 58.42) (end 80.9625 58.42) (width 0.5) (layer F.Cu) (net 13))
 (segment (start 80.01 55.88) (end 78.74 55.88) (width 0.5) (layer F.Cu) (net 14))
 (segment (start 82.55 53.34) (end 80.01 55.88) (width 0.5) (layer F.Cu) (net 14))
 (segment (start 86.425 53.34) (end 82.55 53.34) (width 0.5) (layer F.Cu) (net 14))
 (segment (start 81.915 52.07) (end 80.645 53.34) (width 0.5) (layer F.Cu) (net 15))
 (segment (start 80.645 53.34) (end 78.74 53.34) (width 0.5) (layer F.Cu) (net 15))
 (segment (start 88.9 52.07) (end 81.915 52.07) (width 0.5) (layer F.Cu) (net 15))
 (segment (start 89.535 52.705) (end 88.9 52.07) (width 0.5) (layer F.Cu) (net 15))
 (segment (start 89.535 53.975) (end 89.535 52.705) (width 0.5) (layer F.Cu) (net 15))
 (segment (start 90.17 54.61) (end 89.535 53.975) (width 0.5) (layer F.Cu) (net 15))
 (segment (start 91.375 54.61) (end 90.17 54.61) (width 0.5) (layer F.Cu) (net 15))
 (segment (start 86.995 50.8) (end 78.74 50.8) (width 0.5) (layer F.Cu) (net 16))
 (segment (start 91.375 48.26) (end 88.9 48.26) (width 0.5) (layer F.Cu) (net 16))
 (segment (start 88.9 50.165) (end 88.265 50.8) (width 0.5) (layer F.Cu) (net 16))
 (segment (start 88.265 50.8) (end 86.995 50.8) (width 0.5) (layer F.Cu) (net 16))
 (segment (start 88.9 48.26) (end 88.9 50.165) (width 0.5) (layer F.Cu) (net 16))
 (segment (start 81.28 48.26) (end 78.74 48.26) (width 0.5) (layer F.Cu) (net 17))
 (segment (start 82.55 46.99) (end 81.28 48.26) (width 0.5) (layer F.Cu) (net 17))
 (segment (start 86.425 46.99) (end 82.55 46.99) (width 0.5) (layer F.Cu) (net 17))
 (segment (start 83.82 41.91) (end 86.425 41.91) (width 0.5) (layer F.Cu) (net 18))
 (segment (start 82.8675 41.91) (end 83.82 41.91) (width 0.5) (layer F.Cu) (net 18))
 (segment (start 80.01 44.7675) (end 82.8675 41.91) (width 0.5) (layer F.Cu) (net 18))
 (segment (start 80.01 45.72) (end 80.01 44.7675) (width 0.5) (layer F.Cu) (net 18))
 (segment (start 78.74 45.72) (end 80.01 45.72) (width 0.5) (layer F.Cu) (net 18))
 (segment (start 80.01 43.18) (end 78.74 43.18) (width 0.5) (layer F.Cu) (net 19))
 (segment (start 82.8675 40.3225) (end 80.01 43.18) (width 0.5) (layer F.Cu) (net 19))
 (segment (start 89.535 40.64) (end 89.2175 40.3225) (width 0.5) (layer F.Cu) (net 19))
 (segment (start 89.2175 40.3225) (end 82.8675 40.3225) (width 0.5) (layer F.Cu) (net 19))
 (segment (start 89.535 42.545) (end 89.535 40.64) (width 0.5) (layer F.Cu) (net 19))
 (segment (start 90.17 43.18) (end 89.535 42.545) (width 0.5) (layer F.Cu) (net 19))
 (segment (start 91.375 43.18) (end 90.17 43.18) (width 0.5) (layer F.Cu) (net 19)))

